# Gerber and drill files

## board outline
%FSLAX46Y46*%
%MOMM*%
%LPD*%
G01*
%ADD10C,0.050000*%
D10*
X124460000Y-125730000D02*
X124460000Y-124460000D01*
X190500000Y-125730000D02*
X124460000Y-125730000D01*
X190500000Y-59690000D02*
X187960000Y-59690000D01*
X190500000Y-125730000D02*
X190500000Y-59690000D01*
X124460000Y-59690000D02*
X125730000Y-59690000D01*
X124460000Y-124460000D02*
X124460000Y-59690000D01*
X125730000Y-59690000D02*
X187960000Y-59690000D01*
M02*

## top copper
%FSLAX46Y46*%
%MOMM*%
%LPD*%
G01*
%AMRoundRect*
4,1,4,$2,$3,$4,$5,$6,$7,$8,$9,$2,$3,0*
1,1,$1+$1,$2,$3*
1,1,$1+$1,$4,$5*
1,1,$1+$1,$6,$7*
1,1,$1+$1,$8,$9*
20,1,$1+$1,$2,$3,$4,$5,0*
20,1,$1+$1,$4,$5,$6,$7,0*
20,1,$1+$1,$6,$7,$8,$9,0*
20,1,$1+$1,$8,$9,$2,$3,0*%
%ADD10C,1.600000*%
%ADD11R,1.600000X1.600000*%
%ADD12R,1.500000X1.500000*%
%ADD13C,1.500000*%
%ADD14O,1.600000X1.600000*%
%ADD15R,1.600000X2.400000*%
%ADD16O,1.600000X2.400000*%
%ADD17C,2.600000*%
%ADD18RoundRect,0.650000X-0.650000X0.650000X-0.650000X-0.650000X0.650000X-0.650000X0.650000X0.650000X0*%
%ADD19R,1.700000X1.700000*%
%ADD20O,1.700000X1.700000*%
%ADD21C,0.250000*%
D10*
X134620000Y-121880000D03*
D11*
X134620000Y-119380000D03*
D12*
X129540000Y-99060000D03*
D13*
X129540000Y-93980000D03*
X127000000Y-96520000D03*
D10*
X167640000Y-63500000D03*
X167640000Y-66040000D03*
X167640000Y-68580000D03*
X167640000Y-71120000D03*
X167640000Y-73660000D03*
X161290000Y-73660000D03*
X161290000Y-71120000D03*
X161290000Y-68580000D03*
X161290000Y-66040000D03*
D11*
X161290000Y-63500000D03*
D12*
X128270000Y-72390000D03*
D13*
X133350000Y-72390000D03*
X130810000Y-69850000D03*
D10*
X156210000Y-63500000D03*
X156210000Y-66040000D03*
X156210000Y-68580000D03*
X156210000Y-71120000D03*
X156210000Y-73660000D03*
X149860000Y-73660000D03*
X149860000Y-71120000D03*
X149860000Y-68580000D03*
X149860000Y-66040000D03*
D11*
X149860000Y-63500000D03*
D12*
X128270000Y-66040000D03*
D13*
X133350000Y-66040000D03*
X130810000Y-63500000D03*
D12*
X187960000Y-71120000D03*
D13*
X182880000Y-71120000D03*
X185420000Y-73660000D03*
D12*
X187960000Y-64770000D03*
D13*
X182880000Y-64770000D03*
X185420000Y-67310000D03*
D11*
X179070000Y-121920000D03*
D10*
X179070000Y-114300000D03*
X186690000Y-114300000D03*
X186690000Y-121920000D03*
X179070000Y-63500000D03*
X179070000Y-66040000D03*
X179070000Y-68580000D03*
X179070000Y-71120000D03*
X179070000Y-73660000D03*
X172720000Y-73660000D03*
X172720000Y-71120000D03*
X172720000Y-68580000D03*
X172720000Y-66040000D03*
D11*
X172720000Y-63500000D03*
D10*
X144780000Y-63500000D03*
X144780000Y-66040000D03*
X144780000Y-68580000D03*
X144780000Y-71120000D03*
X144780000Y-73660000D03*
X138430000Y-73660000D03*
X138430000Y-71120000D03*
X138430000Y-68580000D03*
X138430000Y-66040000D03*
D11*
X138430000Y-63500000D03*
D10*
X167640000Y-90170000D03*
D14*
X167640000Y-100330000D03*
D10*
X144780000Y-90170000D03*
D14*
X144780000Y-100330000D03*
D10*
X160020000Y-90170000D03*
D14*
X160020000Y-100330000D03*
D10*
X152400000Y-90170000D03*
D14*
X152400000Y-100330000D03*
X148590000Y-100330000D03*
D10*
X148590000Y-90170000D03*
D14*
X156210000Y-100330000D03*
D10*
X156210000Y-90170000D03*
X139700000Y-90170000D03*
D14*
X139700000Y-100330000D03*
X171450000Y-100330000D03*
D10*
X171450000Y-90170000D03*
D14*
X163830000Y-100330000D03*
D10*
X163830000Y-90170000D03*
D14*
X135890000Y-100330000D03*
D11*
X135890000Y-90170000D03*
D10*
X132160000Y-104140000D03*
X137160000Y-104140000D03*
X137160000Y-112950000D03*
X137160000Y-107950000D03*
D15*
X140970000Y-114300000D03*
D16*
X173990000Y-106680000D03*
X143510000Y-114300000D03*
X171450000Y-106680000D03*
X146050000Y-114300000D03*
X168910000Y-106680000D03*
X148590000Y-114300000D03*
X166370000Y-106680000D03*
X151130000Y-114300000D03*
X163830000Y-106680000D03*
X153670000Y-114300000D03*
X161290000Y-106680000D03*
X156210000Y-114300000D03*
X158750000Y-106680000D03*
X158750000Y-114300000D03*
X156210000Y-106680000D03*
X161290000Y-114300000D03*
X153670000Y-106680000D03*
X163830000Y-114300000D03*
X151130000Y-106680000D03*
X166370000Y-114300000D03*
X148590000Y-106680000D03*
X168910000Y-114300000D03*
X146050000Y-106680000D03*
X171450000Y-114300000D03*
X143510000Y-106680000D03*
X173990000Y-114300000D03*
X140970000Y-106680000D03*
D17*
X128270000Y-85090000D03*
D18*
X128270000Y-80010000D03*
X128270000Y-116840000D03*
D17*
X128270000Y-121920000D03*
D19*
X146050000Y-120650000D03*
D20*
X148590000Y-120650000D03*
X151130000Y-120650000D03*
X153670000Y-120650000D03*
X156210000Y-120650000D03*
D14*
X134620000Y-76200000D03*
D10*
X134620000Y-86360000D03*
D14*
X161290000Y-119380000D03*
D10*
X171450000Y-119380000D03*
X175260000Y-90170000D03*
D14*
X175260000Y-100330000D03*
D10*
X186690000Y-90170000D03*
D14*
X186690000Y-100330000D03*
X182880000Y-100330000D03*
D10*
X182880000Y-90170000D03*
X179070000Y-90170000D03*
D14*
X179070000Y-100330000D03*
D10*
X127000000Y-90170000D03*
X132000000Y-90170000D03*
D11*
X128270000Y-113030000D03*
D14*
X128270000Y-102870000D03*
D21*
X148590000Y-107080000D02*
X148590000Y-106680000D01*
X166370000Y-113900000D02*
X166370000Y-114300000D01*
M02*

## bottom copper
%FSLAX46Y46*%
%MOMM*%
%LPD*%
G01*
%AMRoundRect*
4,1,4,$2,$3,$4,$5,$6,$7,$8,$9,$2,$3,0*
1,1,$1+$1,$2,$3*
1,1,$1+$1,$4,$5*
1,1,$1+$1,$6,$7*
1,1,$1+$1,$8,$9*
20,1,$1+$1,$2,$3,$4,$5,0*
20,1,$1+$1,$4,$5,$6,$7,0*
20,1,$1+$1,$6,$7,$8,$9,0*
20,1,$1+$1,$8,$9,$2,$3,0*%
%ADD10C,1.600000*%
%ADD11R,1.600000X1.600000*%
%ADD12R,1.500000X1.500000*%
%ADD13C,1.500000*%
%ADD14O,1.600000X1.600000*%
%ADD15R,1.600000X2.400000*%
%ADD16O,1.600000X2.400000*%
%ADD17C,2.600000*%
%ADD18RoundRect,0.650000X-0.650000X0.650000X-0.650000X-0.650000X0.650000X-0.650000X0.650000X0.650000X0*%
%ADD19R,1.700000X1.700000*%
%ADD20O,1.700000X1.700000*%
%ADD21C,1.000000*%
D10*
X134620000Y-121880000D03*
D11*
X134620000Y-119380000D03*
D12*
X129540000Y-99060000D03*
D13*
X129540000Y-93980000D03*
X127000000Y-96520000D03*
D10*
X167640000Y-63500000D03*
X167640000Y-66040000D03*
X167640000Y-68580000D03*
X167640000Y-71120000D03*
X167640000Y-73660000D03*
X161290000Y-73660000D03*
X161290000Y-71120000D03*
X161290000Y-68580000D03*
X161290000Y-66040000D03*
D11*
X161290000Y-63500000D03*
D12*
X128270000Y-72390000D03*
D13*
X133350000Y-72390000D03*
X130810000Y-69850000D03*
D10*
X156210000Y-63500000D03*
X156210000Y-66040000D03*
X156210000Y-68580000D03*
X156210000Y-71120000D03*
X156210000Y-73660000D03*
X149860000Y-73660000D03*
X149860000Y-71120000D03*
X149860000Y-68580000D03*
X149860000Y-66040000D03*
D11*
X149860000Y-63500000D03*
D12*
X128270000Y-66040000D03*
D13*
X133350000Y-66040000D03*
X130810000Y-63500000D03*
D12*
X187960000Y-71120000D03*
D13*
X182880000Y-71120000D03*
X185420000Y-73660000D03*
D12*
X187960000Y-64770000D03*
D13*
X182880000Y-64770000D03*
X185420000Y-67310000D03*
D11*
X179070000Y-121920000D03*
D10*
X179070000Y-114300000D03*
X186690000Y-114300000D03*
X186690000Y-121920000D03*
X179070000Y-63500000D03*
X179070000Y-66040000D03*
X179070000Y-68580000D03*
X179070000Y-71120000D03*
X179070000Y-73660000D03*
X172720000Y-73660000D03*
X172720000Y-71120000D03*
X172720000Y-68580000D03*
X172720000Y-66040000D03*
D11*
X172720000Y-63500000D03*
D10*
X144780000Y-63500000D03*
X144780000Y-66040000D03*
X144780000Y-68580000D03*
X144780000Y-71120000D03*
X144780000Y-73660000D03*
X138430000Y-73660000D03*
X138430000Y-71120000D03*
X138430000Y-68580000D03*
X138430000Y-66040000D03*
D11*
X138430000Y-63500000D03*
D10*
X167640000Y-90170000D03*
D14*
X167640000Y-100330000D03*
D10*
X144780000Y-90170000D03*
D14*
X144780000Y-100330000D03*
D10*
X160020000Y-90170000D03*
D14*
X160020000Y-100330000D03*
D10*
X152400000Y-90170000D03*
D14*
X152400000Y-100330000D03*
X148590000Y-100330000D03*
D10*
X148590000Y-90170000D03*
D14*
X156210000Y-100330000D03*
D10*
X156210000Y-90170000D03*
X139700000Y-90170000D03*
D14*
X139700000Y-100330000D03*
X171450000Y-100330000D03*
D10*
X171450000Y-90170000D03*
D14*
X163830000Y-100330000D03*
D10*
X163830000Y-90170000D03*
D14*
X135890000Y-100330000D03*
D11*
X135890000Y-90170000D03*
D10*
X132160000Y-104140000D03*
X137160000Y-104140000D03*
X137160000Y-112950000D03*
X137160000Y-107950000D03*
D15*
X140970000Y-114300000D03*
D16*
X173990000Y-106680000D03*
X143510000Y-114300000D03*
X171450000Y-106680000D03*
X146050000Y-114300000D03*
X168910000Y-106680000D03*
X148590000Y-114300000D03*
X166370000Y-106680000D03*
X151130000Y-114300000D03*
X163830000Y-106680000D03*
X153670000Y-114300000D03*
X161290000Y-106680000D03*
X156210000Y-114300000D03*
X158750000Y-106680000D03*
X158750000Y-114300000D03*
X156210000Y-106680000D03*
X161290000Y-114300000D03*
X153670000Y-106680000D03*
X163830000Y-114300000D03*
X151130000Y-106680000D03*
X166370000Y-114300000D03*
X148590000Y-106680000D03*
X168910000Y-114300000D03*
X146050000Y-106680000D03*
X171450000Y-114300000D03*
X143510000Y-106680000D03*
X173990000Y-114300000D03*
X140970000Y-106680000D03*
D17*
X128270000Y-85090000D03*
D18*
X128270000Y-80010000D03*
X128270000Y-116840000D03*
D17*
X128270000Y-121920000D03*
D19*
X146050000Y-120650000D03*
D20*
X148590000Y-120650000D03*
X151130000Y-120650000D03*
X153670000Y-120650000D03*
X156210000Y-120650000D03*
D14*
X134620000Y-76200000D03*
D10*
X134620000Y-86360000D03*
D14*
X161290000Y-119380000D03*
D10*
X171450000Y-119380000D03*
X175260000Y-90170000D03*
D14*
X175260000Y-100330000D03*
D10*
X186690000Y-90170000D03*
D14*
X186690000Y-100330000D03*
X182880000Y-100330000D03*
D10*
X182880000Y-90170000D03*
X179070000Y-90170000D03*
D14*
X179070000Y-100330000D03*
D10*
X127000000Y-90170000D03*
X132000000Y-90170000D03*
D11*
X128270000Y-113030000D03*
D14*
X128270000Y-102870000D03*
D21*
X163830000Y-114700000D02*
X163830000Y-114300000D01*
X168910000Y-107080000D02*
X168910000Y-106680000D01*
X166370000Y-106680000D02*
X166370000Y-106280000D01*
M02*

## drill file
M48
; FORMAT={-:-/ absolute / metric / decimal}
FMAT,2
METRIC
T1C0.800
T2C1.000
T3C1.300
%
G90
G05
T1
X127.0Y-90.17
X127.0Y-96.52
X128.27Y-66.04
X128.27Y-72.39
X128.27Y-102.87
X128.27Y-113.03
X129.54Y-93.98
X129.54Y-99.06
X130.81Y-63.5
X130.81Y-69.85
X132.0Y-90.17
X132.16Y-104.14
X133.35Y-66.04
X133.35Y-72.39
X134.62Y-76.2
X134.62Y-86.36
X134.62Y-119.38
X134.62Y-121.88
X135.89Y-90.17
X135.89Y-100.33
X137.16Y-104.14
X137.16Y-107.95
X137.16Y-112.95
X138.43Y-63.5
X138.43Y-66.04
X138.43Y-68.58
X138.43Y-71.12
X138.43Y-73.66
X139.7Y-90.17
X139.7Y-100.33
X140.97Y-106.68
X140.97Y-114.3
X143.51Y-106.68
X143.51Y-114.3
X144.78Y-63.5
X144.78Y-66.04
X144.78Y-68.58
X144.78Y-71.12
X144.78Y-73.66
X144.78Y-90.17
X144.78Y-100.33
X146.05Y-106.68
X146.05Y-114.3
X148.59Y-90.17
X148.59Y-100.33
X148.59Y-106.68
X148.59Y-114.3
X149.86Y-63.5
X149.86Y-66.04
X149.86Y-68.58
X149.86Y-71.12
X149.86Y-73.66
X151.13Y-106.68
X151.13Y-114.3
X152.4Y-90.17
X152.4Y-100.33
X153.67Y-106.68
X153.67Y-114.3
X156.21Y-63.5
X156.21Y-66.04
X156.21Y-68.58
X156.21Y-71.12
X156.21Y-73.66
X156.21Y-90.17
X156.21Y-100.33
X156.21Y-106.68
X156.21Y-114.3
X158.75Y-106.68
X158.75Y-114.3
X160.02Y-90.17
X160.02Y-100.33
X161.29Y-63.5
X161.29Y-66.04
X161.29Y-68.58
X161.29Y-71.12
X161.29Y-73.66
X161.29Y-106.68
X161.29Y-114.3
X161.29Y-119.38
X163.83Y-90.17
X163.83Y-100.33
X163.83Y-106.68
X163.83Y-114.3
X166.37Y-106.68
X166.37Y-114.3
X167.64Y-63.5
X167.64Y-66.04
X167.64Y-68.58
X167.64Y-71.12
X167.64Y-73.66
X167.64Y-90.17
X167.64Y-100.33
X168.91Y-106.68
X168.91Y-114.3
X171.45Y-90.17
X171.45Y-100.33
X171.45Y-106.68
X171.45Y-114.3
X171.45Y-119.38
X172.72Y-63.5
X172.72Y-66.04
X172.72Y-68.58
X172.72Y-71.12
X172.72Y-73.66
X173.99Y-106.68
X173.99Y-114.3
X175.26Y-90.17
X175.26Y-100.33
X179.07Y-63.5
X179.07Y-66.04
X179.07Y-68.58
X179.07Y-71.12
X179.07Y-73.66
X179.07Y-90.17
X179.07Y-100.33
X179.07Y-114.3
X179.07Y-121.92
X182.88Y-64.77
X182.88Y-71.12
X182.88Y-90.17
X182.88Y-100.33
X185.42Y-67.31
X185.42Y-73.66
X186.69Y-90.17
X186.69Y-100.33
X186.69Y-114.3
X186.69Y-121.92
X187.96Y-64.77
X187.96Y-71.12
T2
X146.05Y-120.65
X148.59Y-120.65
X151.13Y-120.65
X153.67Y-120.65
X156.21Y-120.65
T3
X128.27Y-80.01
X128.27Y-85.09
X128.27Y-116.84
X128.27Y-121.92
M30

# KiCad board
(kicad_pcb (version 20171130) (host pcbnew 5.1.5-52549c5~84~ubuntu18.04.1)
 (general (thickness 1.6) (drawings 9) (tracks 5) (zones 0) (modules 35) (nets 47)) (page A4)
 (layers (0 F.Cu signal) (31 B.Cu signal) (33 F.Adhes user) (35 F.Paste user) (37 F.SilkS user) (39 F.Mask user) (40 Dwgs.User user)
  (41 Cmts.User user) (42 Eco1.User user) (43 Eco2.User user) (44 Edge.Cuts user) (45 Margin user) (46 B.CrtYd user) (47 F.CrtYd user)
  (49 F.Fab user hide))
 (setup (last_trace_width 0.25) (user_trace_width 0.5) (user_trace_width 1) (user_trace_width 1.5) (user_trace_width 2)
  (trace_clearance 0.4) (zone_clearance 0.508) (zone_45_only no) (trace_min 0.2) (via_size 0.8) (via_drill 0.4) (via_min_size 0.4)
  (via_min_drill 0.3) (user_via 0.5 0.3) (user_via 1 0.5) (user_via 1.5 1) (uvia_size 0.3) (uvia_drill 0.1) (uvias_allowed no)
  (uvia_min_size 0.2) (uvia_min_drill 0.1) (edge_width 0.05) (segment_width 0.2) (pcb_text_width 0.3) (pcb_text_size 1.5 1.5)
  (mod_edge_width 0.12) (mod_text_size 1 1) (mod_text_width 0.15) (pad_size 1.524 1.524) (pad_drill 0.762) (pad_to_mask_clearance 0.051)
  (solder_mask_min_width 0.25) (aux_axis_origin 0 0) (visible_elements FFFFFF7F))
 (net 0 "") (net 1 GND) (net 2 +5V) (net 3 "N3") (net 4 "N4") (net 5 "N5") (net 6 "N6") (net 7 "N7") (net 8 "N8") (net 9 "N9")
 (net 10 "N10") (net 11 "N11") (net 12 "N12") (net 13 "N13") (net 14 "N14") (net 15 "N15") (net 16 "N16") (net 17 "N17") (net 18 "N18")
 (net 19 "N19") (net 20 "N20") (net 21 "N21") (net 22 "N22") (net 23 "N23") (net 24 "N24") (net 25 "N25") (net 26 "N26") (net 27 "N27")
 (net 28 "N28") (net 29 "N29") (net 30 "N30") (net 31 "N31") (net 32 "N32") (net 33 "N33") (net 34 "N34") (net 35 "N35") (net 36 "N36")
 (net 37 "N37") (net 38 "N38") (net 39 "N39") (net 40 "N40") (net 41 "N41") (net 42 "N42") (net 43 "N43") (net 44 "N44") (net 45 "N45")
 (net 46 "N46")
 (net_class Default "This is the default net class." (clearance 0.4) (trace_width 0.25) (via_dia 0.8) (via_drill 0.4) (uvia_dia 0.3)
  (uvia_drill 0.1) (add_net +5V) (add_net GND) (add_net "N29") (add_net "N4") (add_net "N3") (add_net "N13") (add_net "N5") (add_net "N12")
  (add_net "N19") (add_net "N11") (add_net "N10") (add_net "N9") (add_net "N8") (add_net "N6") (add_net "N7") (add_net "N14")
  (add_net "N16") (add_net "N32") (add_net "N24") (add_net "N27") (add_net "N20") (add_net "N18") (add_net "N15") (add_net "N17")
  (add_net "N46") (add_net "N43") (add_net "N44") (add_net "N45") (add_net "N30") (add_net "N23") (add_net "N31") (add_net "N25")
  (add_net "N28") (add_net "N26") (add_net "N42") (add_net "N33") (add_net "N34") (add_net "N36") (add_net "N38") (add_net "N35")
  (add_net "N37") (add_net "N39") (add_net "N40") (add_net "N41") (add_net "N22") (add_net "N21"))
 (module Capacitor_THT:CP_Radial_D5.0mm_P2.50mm (layer F.Cu) (at 134.62 119.38 270)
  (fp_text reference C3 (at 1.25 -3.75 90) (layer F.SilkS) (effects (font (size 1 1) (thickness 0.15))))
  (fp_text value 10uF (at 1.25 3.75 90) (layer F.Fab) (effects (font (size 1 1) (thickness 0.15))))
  (pad 2 thru_hole circle (at 2.5 0 270) (size 1.6 1.6) (drill 0.8) (layers *.Cu *.Mask) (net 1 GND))
  (pad 1 thru_hole rect (at 0 0 270) (size 1.6 1.6) (drill 0.8) (layers *.Cu *.Mask) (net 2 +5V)))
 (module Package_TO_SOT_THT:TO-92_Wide (layer F.Cu) (at 129.54 99.06 90)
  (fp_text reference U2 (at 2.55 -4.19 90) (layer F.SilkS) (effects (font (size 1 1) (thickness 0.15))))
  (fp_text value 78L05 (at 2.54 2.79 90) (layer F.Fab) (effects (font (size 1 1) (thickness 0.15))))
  (pad 1 thru_hole rect (at 0 0 180) (size 1.5 1.5) (drill 0.8) (layers *.Cu *.Mask) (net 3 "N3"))
  (pad 3 thru_hole circle (at 5.08 0 180) (size 1.5 1.5) (drill 0.8) (layers *.Cu *.Mask) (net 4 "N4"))
  (pad 2 thru_hole circle (at 2.54 -2.54 180) (size 1.5 1.5) (drill 0.8) (layers *.Cu *.Mask) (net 1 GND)))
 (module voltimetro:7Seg (layer F.Cu) (at 161.29 63.5)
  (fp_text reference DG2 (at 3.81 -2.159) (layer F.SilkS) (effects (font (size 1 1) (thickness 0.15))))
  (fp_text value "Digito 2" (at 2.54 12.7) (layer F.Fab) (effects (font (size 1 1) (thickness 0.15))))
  (pad 10 thru_hole circle (at 6.35 0) (size 1.6 1.6) (drill 0.8) (layers *.Cu *.Mask) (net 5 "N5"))
  (pad 9 thru_hole circle (at 6.35 2.54) (size 1.6 1.6) (drill 0.8) (layers *.Cu *.Mask) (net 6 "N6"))
  (pad 8 thru_hole circle (at 6.35 5.08) (size 1.6 1.6) (drill 0.8) (layers *.Cu *.Mask) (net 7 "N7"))
  (pad 7 thru_hole circle (at 6.35 7.62) (size 1.6 1.6) (drill 0.8) (layers *.Cu *.Mask) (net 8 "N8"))
  (pad 6 thru_hole circle (at 6.35 10.16) (size 1.6 1.6) (drill 0.8) (layers *.Cu *.Mask) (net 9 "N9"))
  (pad 5 thru_hole circle (at 0 10.16) (size 1.6 1.6) (drill 0.8) (layers *.Cu *.Mask) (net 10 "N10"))
  (pad 4 thru_hole circle (at 0 7.62) (size 1.6 1.6) (drill 0.8) (layers *.Cu *.Mask) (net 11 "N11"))
  (pad 3 thru_hole circle (at 0 5.08) (size 1.6 1.6) (drill 0.8) (layers *.Cu *.Mask) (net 7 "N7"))
  (pad 2 thru_hole circle (at 0 2.54) (size 1.6 1.6) (drill 0.8) (layers *.Cu *.Mask) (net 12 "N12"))
  (pad 1 thru_hole rect (at 0 0) (size 1.6 1.6) (drill 0.8) (layers *.Cu *.Mask) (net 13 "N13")))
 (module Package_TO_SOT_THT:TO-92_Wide (layer F.Cu) (at 128.27 72.39)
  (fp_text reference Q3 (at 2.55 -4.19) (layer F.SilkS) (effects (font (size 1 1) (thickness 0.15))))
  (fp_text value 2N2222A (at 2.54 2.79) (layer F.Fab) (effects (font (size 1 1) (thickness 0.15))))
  (pad 1 thru_hole rect (at 0 0 90) (size 1.5 1.5) (drill 0.8) (layers *.Cu *.Mask) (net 1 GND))
  (pad 3 thru_hole circle (at 5.08 0 90) (size 1.5 1.5) (drill 0.8) (layers *.Cu *.Mask) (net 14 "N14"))
  (pad 2 thru_hole circle (at 2.54 -2.54 90) (size 1.5 1.5) (drill 0.8) (layers *.Cu *.Mask) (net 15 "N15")))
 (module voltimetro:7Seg (layer F.Cu) (at 149.86 63.5)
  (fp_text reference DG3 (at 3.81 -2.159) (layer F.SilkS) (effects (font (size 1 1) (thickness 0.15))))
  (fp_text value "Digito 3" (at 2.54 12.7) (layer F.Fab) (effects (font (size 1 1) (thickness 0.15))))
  (pad 10 thru_hole circle (at 6.35 0) (size 1.6 1.6) (drill 0.8) (layers *.Cu *.Mask) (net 5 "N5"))
  (pad 9 thru_hole circle (at 6.35 2.54) (size 1.6 1.6) (drill 0.8) (layers *.Cu *.Mask) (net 6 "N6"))
  (pad 8 thru_hole circle (at 6.35 5.08) (size 1.6 1.6) (drill 0.8) (layers *.Cu *.Mask) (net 14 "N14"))
  (pad 7 thru_hole circle (at 6.35 7.62) (size 1.6 1.6) (drill 0.8) (layers *.Cu *.Mask) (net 8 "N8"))
  (pad 6 thru_hole circle (at 6.35 10.16) (size 1.6 1.6) (drill 0.8) (layers *.Cu *.Mask) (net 9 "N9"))
  (pad 5 thru_hole circle (at 0 10.16) (size 1.6 1.6) (drill 0.8) (layers *.Cu *.Mask) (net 10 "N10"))
  (pad 4 thru_hole circle (at 0 7.62) (size 1.6 1.6) (drill 0.8) (layers *.Cu *.Mask) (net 11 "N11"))
  (pad 3 thru_hole circle (at 0 5.08) (size 1.6 1.6) (drill 0.8) (layers *.Cu *.Mask) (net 14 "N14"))
  (pad 2 thru_hole circle (at 0 2.54) (size 1.6 1.6) (drill 0.8) (layers *.Cu *.Mask) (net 12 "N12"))
  (pad 1 thru_hole rect (at 0 0) (size 1.6 1.6) (drill 0.8) (layers *.Cu *.Mask) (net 13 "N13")))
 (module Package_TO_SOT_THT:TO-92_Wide (layer F.Cu) (at 128.27 66.04)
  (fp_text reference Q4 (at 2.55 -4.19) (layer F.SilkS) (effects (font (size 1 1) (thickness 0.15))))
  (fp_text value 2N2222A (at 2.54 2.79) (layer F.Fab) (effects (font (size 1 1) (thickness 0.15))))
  (pad 1 thru_hole rect (at 0 0 90) (size 1.5 1.5) (drill 0.8) (layers *.Cu *.Mask) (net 1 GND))
  (pad 3 thru_hole circle (at 5.08 0 90) (size 1.5 1.5) (drill 0.8) (layers *.Cu *.Mask) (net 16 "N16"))
  (pad 2 thru_hole circle (at 2.54 -2.54 90) (size 1.5 1.5) (drill 0.8) (layers *.Cu *.Mask) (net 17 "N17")))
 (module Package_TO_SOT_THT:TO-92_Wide (layer F.Cu) (at 187.96 71.12 180)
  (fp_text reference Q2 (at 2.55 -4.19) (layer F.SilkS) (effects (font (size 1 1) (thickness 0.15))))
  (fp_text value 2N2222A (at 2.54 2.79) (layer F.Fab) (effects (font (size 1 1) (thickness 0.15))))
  (pad 1 thru_hole rect (at 0 0 270) (size 1.5 1.5) (drill 0.8) (layers *.Cu *.Mask) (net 1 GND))
  (pad 3 thru_hole circle (at 5.08 0 270) (size 1.5 1.5) (drill 0.8) (layers *.Cu *.Mask) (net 7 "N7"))
  (pad 2 thru_hole circle (at 2.54 -2.54 270) (size 1.5 1.5) (drill 0.8) (layers *.Cu *.Mask) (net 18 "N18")))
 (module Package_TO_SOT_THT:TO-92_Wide (layer F.Cu) (at 187.96 64.77 180)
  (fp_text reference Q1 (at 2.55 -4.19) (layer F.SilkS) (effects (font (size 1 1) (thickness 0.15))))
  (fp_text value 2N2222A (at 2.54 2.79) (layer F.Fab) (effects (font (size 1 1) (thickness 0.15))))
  (pad 1 thru_hole rect (at 0 0 270) (size 1.5 1.5) (drill 0.8) (layers *.Cu *.Mask) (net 1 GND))
  (pad 3 thru_hole circle (at 5.08 0 270) (size 1.5 1.5) (drill 0.8) (layers *.Cu *.Mask) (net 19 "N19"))
  (pad 2 thru_hole circle (at 2.54 -2.54 270) (size 1.5 1.5) (drill 0.8) (layers *.Cu *.Mask) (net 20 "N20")))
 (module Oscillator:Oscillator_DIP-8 (layer F.Cu) (at 179.07 121.92)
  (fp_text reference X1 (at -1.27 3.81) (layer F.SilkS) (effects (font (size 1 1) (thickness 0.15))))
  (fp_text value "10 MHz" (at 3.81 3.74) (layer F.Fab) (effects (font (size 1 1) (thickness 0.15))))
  (pad 1 thru_hole rect (at 0 0) (size 1.6 1.6) (drill 0.8) (layers *.Cu *.Mask) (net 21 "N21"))
  (pad 8 thru_hole circle (at 0 -7.62) (size 1.6 1.6) (drill 0.8) (layers *.Cu *.Mask) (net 2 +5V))
  (pad 5 thru_hole circle (at 7.62 -7.62) (size 1.6 1.6) (drill 0.8) (layers *.Cu *.Mask) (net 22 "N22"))
  (pad 4 thru_hole circle (at 7.62 0) (size 1.6 1.6) (drill 0.8) (layers *.Cu *.Mask) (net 1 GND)))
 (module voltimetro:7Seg (layer F.Cu) (at 172.72 63.5)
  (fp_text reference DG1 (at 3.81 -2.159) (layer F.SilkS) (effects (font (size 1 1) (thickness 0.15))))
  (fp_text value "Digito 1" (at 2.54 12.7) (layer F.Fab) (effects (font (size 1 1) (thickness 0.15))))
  (pad 10 thru_hole circle (at 6.35 0) (size 1.6 1.6) (drill 0.8) (layers *.Cu *.Mask) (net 5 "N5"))
  (pad 9 thru_hole circle (at 6.35 2.54) (size 1.6 1.6) (drill 0.8) (layers *.Cu *.Mask) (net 6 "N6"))
  (pad 8 thru_hole circle (at 6.35 5.08) (size 1.6 1.6) (drill 0.8) (layers *.Cu *.Mask) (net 19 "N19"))
  (pad 7 thru_hole circle (at 6.35 7.62) (size 1.6 1.6) (drill 0.8) (layers *.Cu *.Mask) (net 8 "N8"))
  (pad 6 thru_hole circle (at 6.35 10.16) (size 1.6 1.6) (drill 0.8) (layers *.Cu *.Mask) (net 9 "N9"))
  (pad 5 thru_hole circle (at 0 10.16) (size 1.6 1.6) (drill 0.8) (layers *.Cu *.Mask) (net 10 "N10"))
  (pad 4 thru_hole circle (at 0 7.62) (size 1.6 1.6) (drill 0.8) (layers *.Cu *.Mask) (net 11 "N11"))
  (pad 3 thru_hole circle (at 0 5.08) (size 1.6 1.6) (drill 0.8) (layers *.Cu *.Mask) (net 19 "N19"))
  (pad 2 thru_hole circle (at 0 2.54) (size 1.6 1.6) (drill 0.8) (layers *.Cu *.Mask) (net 12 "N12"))
  (pad 1 thru_hole rect (at 0 0) (size 1.6 1.6) (drill 0.8) (layers *.Cu *.Mask) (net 13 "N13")))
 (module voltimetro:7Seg (layer F.Cu) (at 138.43 63.5)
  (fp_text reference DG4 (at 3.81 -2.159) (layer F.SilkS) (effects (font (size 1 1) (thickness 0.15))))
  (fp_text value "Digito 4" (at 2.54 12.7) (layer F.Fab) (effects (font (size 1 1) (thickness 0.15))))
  (pad 10 thru_hole circle (at 6.35 0) (size 1.6 1.6) (drill 0.8) (layers *.Cu *.Mask) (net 5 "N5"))
  (pad 9 thru_hole circle (at 6.35 2.54) (size 1.6 1.6) (drill 0.8) (layers *.Cu *.Mask) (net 6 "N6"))
  (pad 8 thru_hole circle (at 6.35 5.08) (size 1.6 1.6) (drill 0.8) (layers *.Cu *.Mask) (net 16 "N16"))
  (pad 7 thru_hole circle (at 6.35 7.62) (size 1.6 1.6) (drill 0.8) (layers *.Cu *.Mask) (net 8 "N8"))
  (pad 6 thru_hole circle (at 6.35 10.16) (size 1.6 1.6) (drill 0.8) (layers *.Cu *.Mask) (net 9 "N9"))
  (pad 5 thru_hole circle (at 0 10.16) (size 1.6 1.6) (drill 0.8) (layers *.Cu *.Mask) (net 10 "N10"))
  (pad 4 thru_hole circle (at 0 7.62) (size 1.6 1.6) (drill 0.8) (layers *.Cu *.Mask) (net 11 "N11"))
  (pad 3 thru_hole circle (at 0 5.08) (size 1.6 1.6) (drill 0.8) (layers *.Cu *.Mask) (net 16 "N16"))
  (pad 2 thru_hole circle (at 0 2.54) (size 1.6 1.6) (drill 0.8) (layers *.Cu *.Mask) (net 12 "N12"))
  (pad 1 thru_hole rect (at 0 0) (size 1.6 1.6) (drill 0.8) (layers *.Cu *.Mask) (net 13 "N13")))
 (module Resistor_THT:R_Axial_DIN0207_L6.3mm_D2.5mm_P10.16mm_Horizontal (layer F.Cu) (at 167.64 90.17 270)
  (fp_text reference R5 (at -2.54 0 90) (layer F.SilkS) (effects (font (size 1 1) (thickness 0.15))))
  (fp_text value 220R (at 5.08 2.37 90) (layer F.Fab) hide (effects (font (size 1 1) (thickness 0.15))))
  (pad 1 thru_hole circle (at 0 0 270) (size 1.6 1.6) (drill 0.8) (layers *.Cu *.Mask) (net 9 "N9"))
  (pad 2 thru_hole oval (at 10.16 0 270) (size 1.6 1.6) (drill 0.8) (layers *.Cu *.Mask) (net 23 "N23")))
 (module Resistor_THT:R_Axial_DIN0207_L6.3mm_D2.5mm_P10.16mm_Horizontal (layer F.Cu) (at 144.78 90.17 270)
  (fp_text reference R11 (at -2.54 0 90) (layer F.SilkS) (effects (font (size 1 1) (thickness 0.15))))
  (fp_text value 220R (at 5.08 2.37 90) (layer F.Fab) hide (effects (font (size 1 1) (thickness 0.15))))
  (pad 1 thru_hole circle (at 0 0 270) (size 1.6 1.6) (drill 0.8) (layers *.Cu *.Mask) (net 10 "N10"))
  (pad 2 thru_hole oval (at 10.16 0 270) (size 1.6 1.6) (drill 0.8) (layers *.Cu *.Mask) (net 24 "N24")))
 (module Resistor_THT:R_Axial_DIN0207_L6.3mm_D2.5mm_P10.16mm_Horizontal (layer F.Cu) (at 160.02 90.17 270)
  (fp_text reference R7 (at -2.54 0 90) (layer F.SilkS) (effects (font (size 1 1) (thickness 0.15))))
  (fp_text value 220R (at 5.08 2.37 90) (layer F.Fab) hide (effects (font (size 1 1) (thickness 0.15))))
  (pad 1 thru_hole circle (at 0 0 270) (size 1.6 1.6) (drill 0.8) (layers *.Cu *.Mask) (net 12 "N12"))
  (pad 2 thru_hole oval (at 10.16 0 270) (size 1.6 1.6) (drill 0.8) (layers *.Cu *.Mask) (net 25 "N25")))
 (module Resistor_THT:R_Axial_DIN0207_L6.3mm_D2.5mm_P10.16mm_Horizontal (layer F.Cu) (at 152.4 90.17 270)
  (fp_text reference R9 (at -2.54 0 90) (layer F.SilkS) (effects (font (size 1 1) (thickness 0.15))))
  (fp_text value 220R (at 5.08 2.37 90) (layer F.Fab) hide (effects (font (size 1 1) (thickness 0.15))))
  (pad 1 thru_hole circle (at 0 0 270) (size 1.6 1.6) (drill 0.8) (layers *.Cu *.Mask) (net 6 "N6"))
  (pad 2 thru_hole oval (at 10.16 0 270) (size 1.6 1.6) (drill 0.8) (layers *.Cu *.Mask) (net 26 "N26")))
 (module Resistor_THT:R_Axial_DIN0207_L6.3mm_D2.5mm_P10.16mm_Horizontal (layer F.Cu) (at 148.59 90.17 270)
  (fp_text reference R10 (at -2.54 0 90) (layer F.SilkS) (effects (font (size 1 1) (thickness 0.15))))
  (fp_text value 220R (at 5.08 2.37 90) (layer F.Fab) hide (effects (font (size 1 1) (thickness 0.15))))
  (pad 2 thru_hole oval (at 10.16 0 270) (size 1.6 1.6) (drill 0.8) (layers *.Cu *.Mask) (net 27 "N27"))
  (pad 1 thru_hole circle (at 0 0 270) (size 1.6 1.6) (drill 0.8) (layers *.Cu *.Mask) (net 5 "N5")))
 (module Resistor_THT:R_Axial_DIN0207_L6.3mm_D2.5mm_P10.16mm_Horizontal (layer F.Cu) (at 156.21 90.17 270)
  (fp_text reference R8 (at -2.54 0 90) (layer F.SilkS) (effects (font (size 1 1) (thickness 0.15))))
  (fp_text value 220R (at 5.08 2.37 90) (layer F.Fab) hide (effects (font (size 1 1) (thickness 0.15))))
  (pad 2 thru_hole oval (at 10.16 0 270) (size 1.6 1.6) (drill 0.8) (layers *.Cu *.Mask) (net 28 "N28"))
  (pad 1 thru_hole circle (at 0 0 270) (size 1.6 1.6) (drill 0.8) (layers *.Cu *.Mask) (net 13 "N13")))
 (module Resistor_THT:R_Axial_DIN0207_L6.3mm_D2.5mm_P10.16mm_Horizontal (layer F.Cu) (at 139.7 90.17 270)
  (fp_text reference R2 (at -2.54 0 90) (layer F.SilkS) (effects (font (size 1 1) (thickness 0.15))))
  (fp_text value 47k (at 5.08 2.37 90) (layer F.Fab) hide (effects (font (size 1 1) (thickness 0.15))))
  (pad 1 thru_hole circle (at 0 0 270) (size 1.6 1.6) (drill 0.8) (layers *.Cu *.Mask) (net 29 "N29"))
  (pad 2 thru_hole oval (at 10.16 0 270) (size 1.6 1.6) (drill 0.8) (layers *.Cu *.Mask) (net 1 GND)))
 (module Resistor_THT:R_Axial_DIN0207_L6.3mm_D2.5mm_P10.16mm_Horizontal (layer F.Cu) (at 171.45 90.17 270)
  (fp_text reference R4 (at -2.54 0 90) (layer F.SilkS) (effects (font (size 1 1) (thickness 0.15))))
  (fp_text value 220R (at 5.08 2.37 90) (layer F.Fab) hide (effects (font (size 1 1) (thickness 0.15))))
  (pad 2 thru_hole oval (at 10.16 0 270) (size 1.6 1.6) (drill 0.8) (layers *.Cu *.Mask) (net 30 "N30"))
  (pad 1 thru_hole circle (at 0 0 270) (size 1.6 1.6) (drill 0.8) (layers *.Cu *.Mask) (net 8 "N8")))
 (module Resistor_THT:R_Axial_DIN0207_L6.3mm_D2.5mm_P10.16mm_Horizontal (layer F.Cu) (at 163.83 90.17 270)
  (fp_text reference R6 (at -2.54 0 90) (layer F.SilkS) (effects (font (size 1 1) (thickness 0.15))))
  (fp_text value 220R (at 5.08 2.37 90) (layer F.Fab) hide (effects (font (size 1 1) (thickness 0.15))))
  (pad 2 thru_hole oval (at 10.16 0 270) (size 1.6 1.6) (drill 0.8) (layers *.Cu *.Mask) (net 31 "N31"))
  (pad 1 thru_hole circle (at 0 0 270) (size 1.6 1.6) (drill 0.8) (layers *.Cu *.Mask) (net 11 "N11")))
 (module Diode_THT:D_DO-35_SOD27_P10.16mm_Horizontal (layer F.Cu) (at 135.89 90.17 270)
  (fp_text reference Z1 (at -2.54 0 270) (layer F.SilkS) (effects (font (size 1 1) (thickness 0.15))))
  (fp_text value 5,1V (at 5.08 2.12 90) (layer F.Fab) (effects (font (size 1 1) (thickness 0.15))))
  (pad 2 thru_hole oval (at 10.16 0 270) (size 1.6 1.6) (drill 0.8) (layers *.Cu *.Mask) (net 1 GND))
  (pad 1 thru_hole rect (at 0 0 270) (size 1.6 1.6) (drill 0.8) (layers *.Cu *.Mask) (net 29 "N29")))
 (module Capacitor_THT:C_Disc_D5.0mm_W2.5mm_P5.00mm (layer F.Cu) (at 137.16 104.14 180)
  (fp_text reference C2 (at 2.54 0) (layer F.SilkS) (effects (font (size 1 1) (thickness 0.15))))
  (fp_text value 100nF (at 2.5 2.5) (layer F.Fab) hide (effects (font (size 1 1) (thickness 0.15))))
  (pad 2 thru_hole circle (at 5 0 180) (size 1.6 1.6) (drill 0.8) (layers *.Cu *.Mask) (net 1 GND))
  (pad 1 thru_hole circle (at 0 0 180) (size 1.6 1.6) (drill 0.8) (layers *.Cu *.Mask) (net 29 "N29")))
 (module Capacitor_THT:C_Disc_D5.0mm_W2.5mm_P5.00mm (layer F.Cu) (at 137.16 107.95 270)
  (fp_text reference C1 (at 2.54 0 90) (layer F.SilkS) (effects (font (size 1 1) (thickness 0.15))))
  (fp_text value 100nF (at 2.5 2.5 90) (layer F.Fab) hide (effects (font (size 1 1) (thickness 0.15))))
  (pad 2 thru_hole circle (at 5 0 270) (size 1.6 1.6) (drill 0.8) (layers *.Cu *.Mask) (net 1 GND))
  (pad 1 thru_hole circle (at 0 0 270) (size 1.6 1.6) (drill 0.8) (layers *.Cu *.Mask) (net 2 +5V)))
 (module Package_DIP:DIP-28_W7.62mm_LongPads (layer F.Cu) (at 140.97 114.3 90)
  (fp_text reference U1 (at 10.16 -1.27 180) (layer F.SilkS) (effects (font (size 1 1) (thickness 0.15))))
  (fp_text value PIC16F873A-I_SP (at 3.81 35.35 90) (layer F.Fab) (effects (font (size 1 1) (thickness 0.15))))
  (pad 1 thru_hole rect (at 0 0 90) (size 2.4 1.6) (drill 0.8) (layers *.Cu *.Mask) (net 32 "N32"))
  (pad 15 thru_hole oval (at 7.62 33.02 90) (size 2.4 1.6) (drill 0.8) (layers *.Cu *.Mask) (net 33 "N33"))
  (pad 2 thru_hole oval (at 0 2.54 90) (size 2.4 1.6) (drill 0.8) (layers *.Cu *.Mask) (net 29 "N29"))
  (pad 16 thru_hole oval (at 7.62 30.48 90) (size 2.4 1.6) (drill 0.8) (layers *.Cu *.Mask) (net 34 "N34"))
  (pad 3 thru_hole oval (at 0 5.08 90) (size 2.4 1.6) (drill 0.8) (layers *.Cu *.Mask) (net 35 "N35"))
  (pad 17 thru_hole oval (at 7.62 27.94 90) (size 2.4 1.6) (drill 0.8) (layers *.Cu *.Mask) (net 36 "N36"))
  (pad 4 thru_hole oval (at 0 7.62 90) (size 2.4 1.6) (drill 0.8) (layers *.Cu *.Mask) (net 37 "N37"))
  (pad 18 thru_hole oval (at 7.62 25.4 90) (size 2.4 1.6) (drill 0.8) (layers *.Cu *.Mask) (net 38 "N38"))
  (pad 5 thru_hole oval (at 0 10.16 90) (size 2.4 1.6) (drill 0.8) (layers *.Cu *.Mask) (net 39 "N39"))
  (pad 19 thru_hole oval (at 7.62 22.86 90) (size 2.4 1.6) (drill 0.8) (layers *.Cu *.Mask) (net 1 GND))
  (pad 6 thru_hole oval (at 0 12.7 90) (size 2.4 1.6) (drill 0.8) (layers *.Cu *.Mask) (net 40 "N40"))
  (pad 20 thru_hole oval (at 7.62 20.32 90) (size 2.4 1.6) (drill 0.8) (layers *.Cu *.Mask) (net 2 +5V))
  (pad 7 thru_hole oval (at 0 15.24 90) (size 2.4 1.6) (drill 0.8) (layers *.Cu *.Mask) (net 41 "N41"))
  (pad 21 thru_hole oval (at 7.62 17.78 90) (size 2.4 1.6) (drill 0.8) (layers *.Cu *.Mask) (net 30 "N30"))
  (pad 8 thru_hole oval (at 0 17.78 90) (size 2.4 1.6) (drill 0.8) (layers *.Cu *.Mask) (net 1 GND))
  (pad 22 thru_hole oval (at 7.62 15.24 90) (size 2.4 1.6) (drill 0.8) (layers *.Cu *.Mask) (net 23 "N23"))
  (pad 9 thru_hole oval (at 0 20.32 90) (size 2.4 1.6) (drill 0.8) (layers *.Cu *.Mask) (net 22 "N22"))
  (pad 23 thru_hole oval (at 7.62 12.7 90) (size 2.4 1.6) (drill 0.8) (layers *.Cu *.Mask) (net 31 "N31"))
  (pad 10 thru_hole oval (at 0 22.86 90) (size 2.4 1.6) (drill 0.8) (layers *.Cu *.Mask) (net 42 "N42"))
  (pad 24 thru_hole oval (at 7.62 10.16 90) (size 2.4 1.6) (drill 0.8) (layers *.Cu *.Mask) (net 25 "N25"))
  (pad 11 thru_hole oval (at 0 25.4 90) (size 2.4 1.6) (drill 0.8) (layers *.Cu *.Mask) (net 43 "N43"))
  (pad 25 thru_hole oval (at 7.62 7.62 90) (size 2.4 1.6) (drill 0.8) (layers *.Cu *.Mask) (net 28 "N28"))
  (pad 12 thru_hole oval (at 0 27.94 90) (size 2.4 1.6) (drill 0.8) (layers *.Cu *.Mask) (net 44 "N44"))
  (pad 26 thru_hole oval (at 7.62 5.08 90) (size 2.4 1.6) (drill 0.8) (layers *.Cu *.Mask) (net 26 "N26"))
  (pad 13 thru_hole oval (at 0 30.48 90) (size 2.4 1.6) (drill 0.8) (layers *.Cu *.Mask) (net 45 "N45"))
  (pad 27 thru_hole oval (at 7.62 2.54 90) (size 2.4 1.6) (drill 0.8) (layers *.Cu *.Mask) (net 27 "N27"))
  (pad 14 thru_hole oval (at 0 33.02 90) (size 2.4 1.6) (drill 0.8) (layers *.Cu *.Mask) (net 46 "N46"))
  (pad 28 thru_hole oval (at 7.62 0 90) (size 2.4 1.6) (drill 0.8) (layers *.Cu *.Mask) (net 24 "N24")))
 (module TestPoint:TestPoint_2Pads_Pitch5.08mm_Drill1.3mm (layer F.Cu) (at 128.27 80.01 270)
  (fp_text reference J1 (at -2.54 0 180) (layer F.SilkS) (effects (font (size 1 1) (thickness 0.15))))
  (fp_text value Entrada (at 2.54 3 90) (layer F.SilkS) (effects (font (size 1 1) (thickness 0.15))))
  (pad 2 thru_hole circle (at 5.08 0 270) (size 2.6 2.6) (drill 1.3) (layers *.Cu *.Mask) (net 1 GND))
  (pad 1 thru_hole roundrect (at 0 0 270) (size 2.6 2.6) (drill 1.3) (layers *.Cu *.Mask) (roundrect_rratio 0.25) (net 4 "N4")))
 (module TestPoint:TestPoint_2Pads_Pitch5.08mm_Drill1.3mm (layer F.Cu) (at 128.27 116.84 270)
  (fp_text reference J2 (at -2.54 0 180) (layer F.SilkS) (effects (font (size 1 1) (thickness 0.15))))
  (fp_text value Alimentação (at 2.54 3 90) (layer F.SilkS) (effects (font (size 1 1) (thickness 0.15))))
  (pad 1 thru_hole roundrect (at 0 0 270) (size 2.6 2.6) (drill 1.3) (layers *.Cu *.Mask) (roundrect_rratio 0.25) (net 2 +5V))
  (pad 2 thru_hole circle (at 5.08 0 270) (size 2.6 2.6) (drill 1.3) (layers *.Cu *.Mask) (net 1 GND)))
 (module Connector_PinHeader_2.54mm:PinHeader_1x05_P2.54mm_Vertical (layer F.Cu) (at 146.05 120.65 90)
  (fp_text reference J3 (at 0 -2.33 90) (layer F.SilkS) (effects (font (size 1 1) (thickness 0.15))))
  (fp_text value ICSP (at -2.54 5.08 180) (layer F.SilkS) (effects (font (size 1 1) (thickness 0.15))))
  (pad 1 thru_hole rect (at 0 0 90) (size 1.7 1.7) (drill 1) (layers *.Cu *.Mask) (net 32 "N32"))
  (pad 2 thru_hole oval (at 0 2.54 90) (size 1.7 1.7) (drill 1) (layers *.Cu *.Mask) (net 2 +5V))
  (pad 3 thru_hole oval (at 0 5.08 90) (size 1.7 1.7) (drill 1) (layers *.Cu *.Mask) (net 1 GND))
  (pad 4 thru_hole oval (at 0 7.62 90) (size 1.7 1.7) (drill 1) (layers *.Cu *.Mask) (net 24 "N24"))
  (pad 5 thru_hole oval (at 0 10.16 90) (size 1.7 1.7) (drill 1) (layers *.Cu *.Mask) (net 27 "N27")))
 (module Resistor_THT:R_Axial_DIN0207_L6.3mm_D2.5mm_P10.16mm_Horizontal (layer F.Cu) (at 134.62 86.36 90)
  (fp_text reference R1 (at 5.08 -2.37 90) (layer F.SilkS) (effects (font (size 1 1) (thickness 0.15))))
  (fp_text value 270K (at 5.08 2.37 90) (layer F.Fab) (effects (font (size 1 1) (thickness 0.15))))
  (pad 2 thru_hole oval (at 10.16 0 90) (size 1.6 1.6) (drill 0.8) (layers *.Cu *.Mask) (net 4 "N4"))
  (pad 1 thru_hole circle (at 0 0 90) (size 1.6 1.6) (drill 0.8) (layers *.Cu *.Mask) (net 29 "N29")))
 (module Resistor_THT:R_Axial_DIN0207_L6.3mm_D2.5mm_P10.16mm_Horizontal (layer F.Cu) (at 171.45 119.38 180)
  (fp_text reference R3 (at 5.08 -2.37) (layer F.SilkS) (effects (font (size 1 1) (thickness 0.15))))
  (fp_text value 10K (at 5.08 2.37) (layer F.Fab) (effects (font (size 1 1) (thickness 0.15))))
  (pad 2 thru_hole oval (at 10.16 0 180) (size 1.6 1.6) (drill 0.8) (layers *.Cu *.Mask) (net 32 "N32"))
  (pad 1 thru_hole circle (at 0 0 180) (size 1.6 1.6) (drill 0.8) (layers *.Cu *.Mask) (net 2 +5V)))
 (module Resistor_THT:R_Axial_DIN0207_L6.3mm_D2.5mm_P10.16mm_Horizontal (layer F.Cu) (at 175.26 90.17 270)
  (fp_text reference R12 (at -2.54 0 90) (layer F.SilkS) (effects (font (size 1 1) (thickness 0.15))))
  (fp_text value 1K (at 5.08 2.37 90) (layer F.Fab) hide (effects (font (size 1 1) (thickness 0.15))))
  (pad 1 thru_hole circle (at 0 0 270) (size 1.6 1.6) (drill 0.8) (layers *.Cu *.Mask) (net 20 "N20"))
  (pad 2 thru_hole oval (at 10.16 0 270) (size 1.6 1.6) (drill 0.8) (layers *.Cu *.Mask) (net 46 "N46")))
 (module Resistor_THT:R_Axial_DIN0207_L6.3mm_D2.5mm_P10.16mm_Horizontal (layer F.Cu) (at 186.69 90.17 270)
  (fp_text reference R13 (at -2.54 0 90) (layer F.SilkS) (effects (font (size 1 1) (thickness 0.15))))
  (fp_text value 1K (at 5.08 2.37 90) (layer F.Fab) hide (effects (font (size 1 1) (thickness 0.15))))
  (pad 1 thru_hole circle (at 0 0 270) (size 1.6 1.6) (drill 0.8) (layers *.Cu *.Mask) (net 17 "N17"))
  (pad 2 thru_hole oval (at 10.16 0 270) (size 1.6 1.6) (drill 0.8) (layers *.Cu *.Mask) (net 43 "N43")))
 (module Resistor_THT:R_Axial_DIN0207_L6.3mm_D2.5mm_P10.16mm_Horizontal (layer F.Cu) (at 182.88 90.17 270)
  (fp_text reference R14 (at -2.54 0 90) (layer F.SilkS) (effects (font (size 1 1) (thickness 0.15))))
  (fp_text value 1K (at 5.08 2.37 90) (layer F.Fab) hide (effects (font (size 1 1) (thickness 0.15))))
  (pad 2 thru_hole oval (at 10.16 0 270) (size 1.6 1.6) (drill 0.8) (layers *.Cu *.Mask) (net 44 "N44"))
  (pad 1 thru_hole circle (at 0 0 270) (size 1.6 1.6) (drill 0.8) (layers *.Cu *.Mask) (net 15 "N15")))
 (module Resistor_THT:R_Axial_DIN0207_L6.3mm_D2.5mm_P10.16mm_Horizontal (layer F.Cu) (at 179.07 90.17 270)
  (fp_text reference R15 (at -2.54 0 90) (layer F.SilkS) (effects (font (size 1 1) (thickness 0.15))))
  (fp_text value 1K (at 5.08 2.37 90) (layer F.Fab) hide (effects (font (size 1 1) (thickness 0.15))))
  (pad 1 thru_hole circle (at 0 0 270) (size 1.6 1.6) (drill 0.8) (layers *.Cu *.Mask) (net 18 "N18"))
  (pad 2 thru_hole oval (at 10.16 0 270) (size 1.6 1.6) (drill 0.8) (layers *.Cu *.Mask) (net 45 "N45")))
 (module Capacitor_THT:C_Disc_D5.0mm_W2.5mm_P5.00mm (layer F.Cu) (at 127 90.17)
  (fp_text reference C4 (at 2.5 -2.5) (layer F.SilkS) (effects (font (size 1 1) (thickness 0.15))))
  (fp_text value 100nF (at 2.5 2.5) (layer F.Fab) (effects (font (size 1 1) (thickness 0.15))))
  (pad 1 thru_hole circle (at 0 0) (size 1.6 1.6) (drill 0.8) (layers *.Cu *.Mask) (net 4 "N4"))
  (pad 2 thru_hole circle (at 5 0) (size 1.6 1.6) (drill 0.8) (layers *.Cu *.Mask) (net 1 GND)))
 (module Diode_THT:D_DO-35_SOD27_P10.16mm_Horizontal (layer F.Cu) (at 128.27 113.03 90)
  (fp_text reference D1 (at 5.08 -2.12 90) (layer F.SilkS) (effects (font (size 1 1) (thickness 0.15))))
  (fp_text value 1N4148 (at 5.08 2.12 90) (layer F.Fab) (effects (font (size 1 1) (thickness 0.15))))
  (pad 1 thru_hole rect (at 0 0 90) (size 1.6 1.6) (drill 0.8) (layers *.Cu *.Mask) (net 2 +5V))
  (pad 2 thru_hole oval (at 10.16 0 90) (size 1.6 1.6) (drill 0.8) (layers *.Cu *.Mask) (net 3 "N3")))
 (gr_line (start 124.46 125.73) (end 124.46 124.46) (layer Edge.Cuts) (width 0.05))
 (gr_line (start 190.5 125.73) (end 124.46 125.73) (layer Edge.Cuts) (width 0.05))
 (gr_line (start 190.5 59.69) (end 187.96 59.69) (layer Edge.Cuts) (width 0.05))
 (gr_line (start 190.5 125.73) (end 190.5 59.69) (layer Edge.Cuts) (width 0.05))
 (gr_line (start 124.46 59.69) (end 125.73 59.69) (layer Edge.Cuts) (width 0.05))
 (gr_line (start 124.46 124.46) (end 124.46 59.69) (layer Edge.Cuts) (width 0.05))
 (gr_line (start 125.73 59.69) (end 187.96 59.69) (layer Edge.Cuts) (width 0.05))
 (segment (start 163.83 114.7) (end 163.83 114.3) (width 1) (layer B.Cu) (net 42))
 (segment (start 168.91 107.08) (end 168.91 106.68) (width 1) (layer B.Cu) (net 36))
 (segment (start 166.37 106.68) (end 166.37 106.28) (width 1) (layer B.Cu) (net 38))
 (segment (start 148.59 107.08) (end 148.59 106.68) (width 0.25) (layer F.Cu) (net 28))
 (segment (start 166.37 113.9) (end 166.37 114.3) (width 0.25) (layer F.Cu) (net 43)))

